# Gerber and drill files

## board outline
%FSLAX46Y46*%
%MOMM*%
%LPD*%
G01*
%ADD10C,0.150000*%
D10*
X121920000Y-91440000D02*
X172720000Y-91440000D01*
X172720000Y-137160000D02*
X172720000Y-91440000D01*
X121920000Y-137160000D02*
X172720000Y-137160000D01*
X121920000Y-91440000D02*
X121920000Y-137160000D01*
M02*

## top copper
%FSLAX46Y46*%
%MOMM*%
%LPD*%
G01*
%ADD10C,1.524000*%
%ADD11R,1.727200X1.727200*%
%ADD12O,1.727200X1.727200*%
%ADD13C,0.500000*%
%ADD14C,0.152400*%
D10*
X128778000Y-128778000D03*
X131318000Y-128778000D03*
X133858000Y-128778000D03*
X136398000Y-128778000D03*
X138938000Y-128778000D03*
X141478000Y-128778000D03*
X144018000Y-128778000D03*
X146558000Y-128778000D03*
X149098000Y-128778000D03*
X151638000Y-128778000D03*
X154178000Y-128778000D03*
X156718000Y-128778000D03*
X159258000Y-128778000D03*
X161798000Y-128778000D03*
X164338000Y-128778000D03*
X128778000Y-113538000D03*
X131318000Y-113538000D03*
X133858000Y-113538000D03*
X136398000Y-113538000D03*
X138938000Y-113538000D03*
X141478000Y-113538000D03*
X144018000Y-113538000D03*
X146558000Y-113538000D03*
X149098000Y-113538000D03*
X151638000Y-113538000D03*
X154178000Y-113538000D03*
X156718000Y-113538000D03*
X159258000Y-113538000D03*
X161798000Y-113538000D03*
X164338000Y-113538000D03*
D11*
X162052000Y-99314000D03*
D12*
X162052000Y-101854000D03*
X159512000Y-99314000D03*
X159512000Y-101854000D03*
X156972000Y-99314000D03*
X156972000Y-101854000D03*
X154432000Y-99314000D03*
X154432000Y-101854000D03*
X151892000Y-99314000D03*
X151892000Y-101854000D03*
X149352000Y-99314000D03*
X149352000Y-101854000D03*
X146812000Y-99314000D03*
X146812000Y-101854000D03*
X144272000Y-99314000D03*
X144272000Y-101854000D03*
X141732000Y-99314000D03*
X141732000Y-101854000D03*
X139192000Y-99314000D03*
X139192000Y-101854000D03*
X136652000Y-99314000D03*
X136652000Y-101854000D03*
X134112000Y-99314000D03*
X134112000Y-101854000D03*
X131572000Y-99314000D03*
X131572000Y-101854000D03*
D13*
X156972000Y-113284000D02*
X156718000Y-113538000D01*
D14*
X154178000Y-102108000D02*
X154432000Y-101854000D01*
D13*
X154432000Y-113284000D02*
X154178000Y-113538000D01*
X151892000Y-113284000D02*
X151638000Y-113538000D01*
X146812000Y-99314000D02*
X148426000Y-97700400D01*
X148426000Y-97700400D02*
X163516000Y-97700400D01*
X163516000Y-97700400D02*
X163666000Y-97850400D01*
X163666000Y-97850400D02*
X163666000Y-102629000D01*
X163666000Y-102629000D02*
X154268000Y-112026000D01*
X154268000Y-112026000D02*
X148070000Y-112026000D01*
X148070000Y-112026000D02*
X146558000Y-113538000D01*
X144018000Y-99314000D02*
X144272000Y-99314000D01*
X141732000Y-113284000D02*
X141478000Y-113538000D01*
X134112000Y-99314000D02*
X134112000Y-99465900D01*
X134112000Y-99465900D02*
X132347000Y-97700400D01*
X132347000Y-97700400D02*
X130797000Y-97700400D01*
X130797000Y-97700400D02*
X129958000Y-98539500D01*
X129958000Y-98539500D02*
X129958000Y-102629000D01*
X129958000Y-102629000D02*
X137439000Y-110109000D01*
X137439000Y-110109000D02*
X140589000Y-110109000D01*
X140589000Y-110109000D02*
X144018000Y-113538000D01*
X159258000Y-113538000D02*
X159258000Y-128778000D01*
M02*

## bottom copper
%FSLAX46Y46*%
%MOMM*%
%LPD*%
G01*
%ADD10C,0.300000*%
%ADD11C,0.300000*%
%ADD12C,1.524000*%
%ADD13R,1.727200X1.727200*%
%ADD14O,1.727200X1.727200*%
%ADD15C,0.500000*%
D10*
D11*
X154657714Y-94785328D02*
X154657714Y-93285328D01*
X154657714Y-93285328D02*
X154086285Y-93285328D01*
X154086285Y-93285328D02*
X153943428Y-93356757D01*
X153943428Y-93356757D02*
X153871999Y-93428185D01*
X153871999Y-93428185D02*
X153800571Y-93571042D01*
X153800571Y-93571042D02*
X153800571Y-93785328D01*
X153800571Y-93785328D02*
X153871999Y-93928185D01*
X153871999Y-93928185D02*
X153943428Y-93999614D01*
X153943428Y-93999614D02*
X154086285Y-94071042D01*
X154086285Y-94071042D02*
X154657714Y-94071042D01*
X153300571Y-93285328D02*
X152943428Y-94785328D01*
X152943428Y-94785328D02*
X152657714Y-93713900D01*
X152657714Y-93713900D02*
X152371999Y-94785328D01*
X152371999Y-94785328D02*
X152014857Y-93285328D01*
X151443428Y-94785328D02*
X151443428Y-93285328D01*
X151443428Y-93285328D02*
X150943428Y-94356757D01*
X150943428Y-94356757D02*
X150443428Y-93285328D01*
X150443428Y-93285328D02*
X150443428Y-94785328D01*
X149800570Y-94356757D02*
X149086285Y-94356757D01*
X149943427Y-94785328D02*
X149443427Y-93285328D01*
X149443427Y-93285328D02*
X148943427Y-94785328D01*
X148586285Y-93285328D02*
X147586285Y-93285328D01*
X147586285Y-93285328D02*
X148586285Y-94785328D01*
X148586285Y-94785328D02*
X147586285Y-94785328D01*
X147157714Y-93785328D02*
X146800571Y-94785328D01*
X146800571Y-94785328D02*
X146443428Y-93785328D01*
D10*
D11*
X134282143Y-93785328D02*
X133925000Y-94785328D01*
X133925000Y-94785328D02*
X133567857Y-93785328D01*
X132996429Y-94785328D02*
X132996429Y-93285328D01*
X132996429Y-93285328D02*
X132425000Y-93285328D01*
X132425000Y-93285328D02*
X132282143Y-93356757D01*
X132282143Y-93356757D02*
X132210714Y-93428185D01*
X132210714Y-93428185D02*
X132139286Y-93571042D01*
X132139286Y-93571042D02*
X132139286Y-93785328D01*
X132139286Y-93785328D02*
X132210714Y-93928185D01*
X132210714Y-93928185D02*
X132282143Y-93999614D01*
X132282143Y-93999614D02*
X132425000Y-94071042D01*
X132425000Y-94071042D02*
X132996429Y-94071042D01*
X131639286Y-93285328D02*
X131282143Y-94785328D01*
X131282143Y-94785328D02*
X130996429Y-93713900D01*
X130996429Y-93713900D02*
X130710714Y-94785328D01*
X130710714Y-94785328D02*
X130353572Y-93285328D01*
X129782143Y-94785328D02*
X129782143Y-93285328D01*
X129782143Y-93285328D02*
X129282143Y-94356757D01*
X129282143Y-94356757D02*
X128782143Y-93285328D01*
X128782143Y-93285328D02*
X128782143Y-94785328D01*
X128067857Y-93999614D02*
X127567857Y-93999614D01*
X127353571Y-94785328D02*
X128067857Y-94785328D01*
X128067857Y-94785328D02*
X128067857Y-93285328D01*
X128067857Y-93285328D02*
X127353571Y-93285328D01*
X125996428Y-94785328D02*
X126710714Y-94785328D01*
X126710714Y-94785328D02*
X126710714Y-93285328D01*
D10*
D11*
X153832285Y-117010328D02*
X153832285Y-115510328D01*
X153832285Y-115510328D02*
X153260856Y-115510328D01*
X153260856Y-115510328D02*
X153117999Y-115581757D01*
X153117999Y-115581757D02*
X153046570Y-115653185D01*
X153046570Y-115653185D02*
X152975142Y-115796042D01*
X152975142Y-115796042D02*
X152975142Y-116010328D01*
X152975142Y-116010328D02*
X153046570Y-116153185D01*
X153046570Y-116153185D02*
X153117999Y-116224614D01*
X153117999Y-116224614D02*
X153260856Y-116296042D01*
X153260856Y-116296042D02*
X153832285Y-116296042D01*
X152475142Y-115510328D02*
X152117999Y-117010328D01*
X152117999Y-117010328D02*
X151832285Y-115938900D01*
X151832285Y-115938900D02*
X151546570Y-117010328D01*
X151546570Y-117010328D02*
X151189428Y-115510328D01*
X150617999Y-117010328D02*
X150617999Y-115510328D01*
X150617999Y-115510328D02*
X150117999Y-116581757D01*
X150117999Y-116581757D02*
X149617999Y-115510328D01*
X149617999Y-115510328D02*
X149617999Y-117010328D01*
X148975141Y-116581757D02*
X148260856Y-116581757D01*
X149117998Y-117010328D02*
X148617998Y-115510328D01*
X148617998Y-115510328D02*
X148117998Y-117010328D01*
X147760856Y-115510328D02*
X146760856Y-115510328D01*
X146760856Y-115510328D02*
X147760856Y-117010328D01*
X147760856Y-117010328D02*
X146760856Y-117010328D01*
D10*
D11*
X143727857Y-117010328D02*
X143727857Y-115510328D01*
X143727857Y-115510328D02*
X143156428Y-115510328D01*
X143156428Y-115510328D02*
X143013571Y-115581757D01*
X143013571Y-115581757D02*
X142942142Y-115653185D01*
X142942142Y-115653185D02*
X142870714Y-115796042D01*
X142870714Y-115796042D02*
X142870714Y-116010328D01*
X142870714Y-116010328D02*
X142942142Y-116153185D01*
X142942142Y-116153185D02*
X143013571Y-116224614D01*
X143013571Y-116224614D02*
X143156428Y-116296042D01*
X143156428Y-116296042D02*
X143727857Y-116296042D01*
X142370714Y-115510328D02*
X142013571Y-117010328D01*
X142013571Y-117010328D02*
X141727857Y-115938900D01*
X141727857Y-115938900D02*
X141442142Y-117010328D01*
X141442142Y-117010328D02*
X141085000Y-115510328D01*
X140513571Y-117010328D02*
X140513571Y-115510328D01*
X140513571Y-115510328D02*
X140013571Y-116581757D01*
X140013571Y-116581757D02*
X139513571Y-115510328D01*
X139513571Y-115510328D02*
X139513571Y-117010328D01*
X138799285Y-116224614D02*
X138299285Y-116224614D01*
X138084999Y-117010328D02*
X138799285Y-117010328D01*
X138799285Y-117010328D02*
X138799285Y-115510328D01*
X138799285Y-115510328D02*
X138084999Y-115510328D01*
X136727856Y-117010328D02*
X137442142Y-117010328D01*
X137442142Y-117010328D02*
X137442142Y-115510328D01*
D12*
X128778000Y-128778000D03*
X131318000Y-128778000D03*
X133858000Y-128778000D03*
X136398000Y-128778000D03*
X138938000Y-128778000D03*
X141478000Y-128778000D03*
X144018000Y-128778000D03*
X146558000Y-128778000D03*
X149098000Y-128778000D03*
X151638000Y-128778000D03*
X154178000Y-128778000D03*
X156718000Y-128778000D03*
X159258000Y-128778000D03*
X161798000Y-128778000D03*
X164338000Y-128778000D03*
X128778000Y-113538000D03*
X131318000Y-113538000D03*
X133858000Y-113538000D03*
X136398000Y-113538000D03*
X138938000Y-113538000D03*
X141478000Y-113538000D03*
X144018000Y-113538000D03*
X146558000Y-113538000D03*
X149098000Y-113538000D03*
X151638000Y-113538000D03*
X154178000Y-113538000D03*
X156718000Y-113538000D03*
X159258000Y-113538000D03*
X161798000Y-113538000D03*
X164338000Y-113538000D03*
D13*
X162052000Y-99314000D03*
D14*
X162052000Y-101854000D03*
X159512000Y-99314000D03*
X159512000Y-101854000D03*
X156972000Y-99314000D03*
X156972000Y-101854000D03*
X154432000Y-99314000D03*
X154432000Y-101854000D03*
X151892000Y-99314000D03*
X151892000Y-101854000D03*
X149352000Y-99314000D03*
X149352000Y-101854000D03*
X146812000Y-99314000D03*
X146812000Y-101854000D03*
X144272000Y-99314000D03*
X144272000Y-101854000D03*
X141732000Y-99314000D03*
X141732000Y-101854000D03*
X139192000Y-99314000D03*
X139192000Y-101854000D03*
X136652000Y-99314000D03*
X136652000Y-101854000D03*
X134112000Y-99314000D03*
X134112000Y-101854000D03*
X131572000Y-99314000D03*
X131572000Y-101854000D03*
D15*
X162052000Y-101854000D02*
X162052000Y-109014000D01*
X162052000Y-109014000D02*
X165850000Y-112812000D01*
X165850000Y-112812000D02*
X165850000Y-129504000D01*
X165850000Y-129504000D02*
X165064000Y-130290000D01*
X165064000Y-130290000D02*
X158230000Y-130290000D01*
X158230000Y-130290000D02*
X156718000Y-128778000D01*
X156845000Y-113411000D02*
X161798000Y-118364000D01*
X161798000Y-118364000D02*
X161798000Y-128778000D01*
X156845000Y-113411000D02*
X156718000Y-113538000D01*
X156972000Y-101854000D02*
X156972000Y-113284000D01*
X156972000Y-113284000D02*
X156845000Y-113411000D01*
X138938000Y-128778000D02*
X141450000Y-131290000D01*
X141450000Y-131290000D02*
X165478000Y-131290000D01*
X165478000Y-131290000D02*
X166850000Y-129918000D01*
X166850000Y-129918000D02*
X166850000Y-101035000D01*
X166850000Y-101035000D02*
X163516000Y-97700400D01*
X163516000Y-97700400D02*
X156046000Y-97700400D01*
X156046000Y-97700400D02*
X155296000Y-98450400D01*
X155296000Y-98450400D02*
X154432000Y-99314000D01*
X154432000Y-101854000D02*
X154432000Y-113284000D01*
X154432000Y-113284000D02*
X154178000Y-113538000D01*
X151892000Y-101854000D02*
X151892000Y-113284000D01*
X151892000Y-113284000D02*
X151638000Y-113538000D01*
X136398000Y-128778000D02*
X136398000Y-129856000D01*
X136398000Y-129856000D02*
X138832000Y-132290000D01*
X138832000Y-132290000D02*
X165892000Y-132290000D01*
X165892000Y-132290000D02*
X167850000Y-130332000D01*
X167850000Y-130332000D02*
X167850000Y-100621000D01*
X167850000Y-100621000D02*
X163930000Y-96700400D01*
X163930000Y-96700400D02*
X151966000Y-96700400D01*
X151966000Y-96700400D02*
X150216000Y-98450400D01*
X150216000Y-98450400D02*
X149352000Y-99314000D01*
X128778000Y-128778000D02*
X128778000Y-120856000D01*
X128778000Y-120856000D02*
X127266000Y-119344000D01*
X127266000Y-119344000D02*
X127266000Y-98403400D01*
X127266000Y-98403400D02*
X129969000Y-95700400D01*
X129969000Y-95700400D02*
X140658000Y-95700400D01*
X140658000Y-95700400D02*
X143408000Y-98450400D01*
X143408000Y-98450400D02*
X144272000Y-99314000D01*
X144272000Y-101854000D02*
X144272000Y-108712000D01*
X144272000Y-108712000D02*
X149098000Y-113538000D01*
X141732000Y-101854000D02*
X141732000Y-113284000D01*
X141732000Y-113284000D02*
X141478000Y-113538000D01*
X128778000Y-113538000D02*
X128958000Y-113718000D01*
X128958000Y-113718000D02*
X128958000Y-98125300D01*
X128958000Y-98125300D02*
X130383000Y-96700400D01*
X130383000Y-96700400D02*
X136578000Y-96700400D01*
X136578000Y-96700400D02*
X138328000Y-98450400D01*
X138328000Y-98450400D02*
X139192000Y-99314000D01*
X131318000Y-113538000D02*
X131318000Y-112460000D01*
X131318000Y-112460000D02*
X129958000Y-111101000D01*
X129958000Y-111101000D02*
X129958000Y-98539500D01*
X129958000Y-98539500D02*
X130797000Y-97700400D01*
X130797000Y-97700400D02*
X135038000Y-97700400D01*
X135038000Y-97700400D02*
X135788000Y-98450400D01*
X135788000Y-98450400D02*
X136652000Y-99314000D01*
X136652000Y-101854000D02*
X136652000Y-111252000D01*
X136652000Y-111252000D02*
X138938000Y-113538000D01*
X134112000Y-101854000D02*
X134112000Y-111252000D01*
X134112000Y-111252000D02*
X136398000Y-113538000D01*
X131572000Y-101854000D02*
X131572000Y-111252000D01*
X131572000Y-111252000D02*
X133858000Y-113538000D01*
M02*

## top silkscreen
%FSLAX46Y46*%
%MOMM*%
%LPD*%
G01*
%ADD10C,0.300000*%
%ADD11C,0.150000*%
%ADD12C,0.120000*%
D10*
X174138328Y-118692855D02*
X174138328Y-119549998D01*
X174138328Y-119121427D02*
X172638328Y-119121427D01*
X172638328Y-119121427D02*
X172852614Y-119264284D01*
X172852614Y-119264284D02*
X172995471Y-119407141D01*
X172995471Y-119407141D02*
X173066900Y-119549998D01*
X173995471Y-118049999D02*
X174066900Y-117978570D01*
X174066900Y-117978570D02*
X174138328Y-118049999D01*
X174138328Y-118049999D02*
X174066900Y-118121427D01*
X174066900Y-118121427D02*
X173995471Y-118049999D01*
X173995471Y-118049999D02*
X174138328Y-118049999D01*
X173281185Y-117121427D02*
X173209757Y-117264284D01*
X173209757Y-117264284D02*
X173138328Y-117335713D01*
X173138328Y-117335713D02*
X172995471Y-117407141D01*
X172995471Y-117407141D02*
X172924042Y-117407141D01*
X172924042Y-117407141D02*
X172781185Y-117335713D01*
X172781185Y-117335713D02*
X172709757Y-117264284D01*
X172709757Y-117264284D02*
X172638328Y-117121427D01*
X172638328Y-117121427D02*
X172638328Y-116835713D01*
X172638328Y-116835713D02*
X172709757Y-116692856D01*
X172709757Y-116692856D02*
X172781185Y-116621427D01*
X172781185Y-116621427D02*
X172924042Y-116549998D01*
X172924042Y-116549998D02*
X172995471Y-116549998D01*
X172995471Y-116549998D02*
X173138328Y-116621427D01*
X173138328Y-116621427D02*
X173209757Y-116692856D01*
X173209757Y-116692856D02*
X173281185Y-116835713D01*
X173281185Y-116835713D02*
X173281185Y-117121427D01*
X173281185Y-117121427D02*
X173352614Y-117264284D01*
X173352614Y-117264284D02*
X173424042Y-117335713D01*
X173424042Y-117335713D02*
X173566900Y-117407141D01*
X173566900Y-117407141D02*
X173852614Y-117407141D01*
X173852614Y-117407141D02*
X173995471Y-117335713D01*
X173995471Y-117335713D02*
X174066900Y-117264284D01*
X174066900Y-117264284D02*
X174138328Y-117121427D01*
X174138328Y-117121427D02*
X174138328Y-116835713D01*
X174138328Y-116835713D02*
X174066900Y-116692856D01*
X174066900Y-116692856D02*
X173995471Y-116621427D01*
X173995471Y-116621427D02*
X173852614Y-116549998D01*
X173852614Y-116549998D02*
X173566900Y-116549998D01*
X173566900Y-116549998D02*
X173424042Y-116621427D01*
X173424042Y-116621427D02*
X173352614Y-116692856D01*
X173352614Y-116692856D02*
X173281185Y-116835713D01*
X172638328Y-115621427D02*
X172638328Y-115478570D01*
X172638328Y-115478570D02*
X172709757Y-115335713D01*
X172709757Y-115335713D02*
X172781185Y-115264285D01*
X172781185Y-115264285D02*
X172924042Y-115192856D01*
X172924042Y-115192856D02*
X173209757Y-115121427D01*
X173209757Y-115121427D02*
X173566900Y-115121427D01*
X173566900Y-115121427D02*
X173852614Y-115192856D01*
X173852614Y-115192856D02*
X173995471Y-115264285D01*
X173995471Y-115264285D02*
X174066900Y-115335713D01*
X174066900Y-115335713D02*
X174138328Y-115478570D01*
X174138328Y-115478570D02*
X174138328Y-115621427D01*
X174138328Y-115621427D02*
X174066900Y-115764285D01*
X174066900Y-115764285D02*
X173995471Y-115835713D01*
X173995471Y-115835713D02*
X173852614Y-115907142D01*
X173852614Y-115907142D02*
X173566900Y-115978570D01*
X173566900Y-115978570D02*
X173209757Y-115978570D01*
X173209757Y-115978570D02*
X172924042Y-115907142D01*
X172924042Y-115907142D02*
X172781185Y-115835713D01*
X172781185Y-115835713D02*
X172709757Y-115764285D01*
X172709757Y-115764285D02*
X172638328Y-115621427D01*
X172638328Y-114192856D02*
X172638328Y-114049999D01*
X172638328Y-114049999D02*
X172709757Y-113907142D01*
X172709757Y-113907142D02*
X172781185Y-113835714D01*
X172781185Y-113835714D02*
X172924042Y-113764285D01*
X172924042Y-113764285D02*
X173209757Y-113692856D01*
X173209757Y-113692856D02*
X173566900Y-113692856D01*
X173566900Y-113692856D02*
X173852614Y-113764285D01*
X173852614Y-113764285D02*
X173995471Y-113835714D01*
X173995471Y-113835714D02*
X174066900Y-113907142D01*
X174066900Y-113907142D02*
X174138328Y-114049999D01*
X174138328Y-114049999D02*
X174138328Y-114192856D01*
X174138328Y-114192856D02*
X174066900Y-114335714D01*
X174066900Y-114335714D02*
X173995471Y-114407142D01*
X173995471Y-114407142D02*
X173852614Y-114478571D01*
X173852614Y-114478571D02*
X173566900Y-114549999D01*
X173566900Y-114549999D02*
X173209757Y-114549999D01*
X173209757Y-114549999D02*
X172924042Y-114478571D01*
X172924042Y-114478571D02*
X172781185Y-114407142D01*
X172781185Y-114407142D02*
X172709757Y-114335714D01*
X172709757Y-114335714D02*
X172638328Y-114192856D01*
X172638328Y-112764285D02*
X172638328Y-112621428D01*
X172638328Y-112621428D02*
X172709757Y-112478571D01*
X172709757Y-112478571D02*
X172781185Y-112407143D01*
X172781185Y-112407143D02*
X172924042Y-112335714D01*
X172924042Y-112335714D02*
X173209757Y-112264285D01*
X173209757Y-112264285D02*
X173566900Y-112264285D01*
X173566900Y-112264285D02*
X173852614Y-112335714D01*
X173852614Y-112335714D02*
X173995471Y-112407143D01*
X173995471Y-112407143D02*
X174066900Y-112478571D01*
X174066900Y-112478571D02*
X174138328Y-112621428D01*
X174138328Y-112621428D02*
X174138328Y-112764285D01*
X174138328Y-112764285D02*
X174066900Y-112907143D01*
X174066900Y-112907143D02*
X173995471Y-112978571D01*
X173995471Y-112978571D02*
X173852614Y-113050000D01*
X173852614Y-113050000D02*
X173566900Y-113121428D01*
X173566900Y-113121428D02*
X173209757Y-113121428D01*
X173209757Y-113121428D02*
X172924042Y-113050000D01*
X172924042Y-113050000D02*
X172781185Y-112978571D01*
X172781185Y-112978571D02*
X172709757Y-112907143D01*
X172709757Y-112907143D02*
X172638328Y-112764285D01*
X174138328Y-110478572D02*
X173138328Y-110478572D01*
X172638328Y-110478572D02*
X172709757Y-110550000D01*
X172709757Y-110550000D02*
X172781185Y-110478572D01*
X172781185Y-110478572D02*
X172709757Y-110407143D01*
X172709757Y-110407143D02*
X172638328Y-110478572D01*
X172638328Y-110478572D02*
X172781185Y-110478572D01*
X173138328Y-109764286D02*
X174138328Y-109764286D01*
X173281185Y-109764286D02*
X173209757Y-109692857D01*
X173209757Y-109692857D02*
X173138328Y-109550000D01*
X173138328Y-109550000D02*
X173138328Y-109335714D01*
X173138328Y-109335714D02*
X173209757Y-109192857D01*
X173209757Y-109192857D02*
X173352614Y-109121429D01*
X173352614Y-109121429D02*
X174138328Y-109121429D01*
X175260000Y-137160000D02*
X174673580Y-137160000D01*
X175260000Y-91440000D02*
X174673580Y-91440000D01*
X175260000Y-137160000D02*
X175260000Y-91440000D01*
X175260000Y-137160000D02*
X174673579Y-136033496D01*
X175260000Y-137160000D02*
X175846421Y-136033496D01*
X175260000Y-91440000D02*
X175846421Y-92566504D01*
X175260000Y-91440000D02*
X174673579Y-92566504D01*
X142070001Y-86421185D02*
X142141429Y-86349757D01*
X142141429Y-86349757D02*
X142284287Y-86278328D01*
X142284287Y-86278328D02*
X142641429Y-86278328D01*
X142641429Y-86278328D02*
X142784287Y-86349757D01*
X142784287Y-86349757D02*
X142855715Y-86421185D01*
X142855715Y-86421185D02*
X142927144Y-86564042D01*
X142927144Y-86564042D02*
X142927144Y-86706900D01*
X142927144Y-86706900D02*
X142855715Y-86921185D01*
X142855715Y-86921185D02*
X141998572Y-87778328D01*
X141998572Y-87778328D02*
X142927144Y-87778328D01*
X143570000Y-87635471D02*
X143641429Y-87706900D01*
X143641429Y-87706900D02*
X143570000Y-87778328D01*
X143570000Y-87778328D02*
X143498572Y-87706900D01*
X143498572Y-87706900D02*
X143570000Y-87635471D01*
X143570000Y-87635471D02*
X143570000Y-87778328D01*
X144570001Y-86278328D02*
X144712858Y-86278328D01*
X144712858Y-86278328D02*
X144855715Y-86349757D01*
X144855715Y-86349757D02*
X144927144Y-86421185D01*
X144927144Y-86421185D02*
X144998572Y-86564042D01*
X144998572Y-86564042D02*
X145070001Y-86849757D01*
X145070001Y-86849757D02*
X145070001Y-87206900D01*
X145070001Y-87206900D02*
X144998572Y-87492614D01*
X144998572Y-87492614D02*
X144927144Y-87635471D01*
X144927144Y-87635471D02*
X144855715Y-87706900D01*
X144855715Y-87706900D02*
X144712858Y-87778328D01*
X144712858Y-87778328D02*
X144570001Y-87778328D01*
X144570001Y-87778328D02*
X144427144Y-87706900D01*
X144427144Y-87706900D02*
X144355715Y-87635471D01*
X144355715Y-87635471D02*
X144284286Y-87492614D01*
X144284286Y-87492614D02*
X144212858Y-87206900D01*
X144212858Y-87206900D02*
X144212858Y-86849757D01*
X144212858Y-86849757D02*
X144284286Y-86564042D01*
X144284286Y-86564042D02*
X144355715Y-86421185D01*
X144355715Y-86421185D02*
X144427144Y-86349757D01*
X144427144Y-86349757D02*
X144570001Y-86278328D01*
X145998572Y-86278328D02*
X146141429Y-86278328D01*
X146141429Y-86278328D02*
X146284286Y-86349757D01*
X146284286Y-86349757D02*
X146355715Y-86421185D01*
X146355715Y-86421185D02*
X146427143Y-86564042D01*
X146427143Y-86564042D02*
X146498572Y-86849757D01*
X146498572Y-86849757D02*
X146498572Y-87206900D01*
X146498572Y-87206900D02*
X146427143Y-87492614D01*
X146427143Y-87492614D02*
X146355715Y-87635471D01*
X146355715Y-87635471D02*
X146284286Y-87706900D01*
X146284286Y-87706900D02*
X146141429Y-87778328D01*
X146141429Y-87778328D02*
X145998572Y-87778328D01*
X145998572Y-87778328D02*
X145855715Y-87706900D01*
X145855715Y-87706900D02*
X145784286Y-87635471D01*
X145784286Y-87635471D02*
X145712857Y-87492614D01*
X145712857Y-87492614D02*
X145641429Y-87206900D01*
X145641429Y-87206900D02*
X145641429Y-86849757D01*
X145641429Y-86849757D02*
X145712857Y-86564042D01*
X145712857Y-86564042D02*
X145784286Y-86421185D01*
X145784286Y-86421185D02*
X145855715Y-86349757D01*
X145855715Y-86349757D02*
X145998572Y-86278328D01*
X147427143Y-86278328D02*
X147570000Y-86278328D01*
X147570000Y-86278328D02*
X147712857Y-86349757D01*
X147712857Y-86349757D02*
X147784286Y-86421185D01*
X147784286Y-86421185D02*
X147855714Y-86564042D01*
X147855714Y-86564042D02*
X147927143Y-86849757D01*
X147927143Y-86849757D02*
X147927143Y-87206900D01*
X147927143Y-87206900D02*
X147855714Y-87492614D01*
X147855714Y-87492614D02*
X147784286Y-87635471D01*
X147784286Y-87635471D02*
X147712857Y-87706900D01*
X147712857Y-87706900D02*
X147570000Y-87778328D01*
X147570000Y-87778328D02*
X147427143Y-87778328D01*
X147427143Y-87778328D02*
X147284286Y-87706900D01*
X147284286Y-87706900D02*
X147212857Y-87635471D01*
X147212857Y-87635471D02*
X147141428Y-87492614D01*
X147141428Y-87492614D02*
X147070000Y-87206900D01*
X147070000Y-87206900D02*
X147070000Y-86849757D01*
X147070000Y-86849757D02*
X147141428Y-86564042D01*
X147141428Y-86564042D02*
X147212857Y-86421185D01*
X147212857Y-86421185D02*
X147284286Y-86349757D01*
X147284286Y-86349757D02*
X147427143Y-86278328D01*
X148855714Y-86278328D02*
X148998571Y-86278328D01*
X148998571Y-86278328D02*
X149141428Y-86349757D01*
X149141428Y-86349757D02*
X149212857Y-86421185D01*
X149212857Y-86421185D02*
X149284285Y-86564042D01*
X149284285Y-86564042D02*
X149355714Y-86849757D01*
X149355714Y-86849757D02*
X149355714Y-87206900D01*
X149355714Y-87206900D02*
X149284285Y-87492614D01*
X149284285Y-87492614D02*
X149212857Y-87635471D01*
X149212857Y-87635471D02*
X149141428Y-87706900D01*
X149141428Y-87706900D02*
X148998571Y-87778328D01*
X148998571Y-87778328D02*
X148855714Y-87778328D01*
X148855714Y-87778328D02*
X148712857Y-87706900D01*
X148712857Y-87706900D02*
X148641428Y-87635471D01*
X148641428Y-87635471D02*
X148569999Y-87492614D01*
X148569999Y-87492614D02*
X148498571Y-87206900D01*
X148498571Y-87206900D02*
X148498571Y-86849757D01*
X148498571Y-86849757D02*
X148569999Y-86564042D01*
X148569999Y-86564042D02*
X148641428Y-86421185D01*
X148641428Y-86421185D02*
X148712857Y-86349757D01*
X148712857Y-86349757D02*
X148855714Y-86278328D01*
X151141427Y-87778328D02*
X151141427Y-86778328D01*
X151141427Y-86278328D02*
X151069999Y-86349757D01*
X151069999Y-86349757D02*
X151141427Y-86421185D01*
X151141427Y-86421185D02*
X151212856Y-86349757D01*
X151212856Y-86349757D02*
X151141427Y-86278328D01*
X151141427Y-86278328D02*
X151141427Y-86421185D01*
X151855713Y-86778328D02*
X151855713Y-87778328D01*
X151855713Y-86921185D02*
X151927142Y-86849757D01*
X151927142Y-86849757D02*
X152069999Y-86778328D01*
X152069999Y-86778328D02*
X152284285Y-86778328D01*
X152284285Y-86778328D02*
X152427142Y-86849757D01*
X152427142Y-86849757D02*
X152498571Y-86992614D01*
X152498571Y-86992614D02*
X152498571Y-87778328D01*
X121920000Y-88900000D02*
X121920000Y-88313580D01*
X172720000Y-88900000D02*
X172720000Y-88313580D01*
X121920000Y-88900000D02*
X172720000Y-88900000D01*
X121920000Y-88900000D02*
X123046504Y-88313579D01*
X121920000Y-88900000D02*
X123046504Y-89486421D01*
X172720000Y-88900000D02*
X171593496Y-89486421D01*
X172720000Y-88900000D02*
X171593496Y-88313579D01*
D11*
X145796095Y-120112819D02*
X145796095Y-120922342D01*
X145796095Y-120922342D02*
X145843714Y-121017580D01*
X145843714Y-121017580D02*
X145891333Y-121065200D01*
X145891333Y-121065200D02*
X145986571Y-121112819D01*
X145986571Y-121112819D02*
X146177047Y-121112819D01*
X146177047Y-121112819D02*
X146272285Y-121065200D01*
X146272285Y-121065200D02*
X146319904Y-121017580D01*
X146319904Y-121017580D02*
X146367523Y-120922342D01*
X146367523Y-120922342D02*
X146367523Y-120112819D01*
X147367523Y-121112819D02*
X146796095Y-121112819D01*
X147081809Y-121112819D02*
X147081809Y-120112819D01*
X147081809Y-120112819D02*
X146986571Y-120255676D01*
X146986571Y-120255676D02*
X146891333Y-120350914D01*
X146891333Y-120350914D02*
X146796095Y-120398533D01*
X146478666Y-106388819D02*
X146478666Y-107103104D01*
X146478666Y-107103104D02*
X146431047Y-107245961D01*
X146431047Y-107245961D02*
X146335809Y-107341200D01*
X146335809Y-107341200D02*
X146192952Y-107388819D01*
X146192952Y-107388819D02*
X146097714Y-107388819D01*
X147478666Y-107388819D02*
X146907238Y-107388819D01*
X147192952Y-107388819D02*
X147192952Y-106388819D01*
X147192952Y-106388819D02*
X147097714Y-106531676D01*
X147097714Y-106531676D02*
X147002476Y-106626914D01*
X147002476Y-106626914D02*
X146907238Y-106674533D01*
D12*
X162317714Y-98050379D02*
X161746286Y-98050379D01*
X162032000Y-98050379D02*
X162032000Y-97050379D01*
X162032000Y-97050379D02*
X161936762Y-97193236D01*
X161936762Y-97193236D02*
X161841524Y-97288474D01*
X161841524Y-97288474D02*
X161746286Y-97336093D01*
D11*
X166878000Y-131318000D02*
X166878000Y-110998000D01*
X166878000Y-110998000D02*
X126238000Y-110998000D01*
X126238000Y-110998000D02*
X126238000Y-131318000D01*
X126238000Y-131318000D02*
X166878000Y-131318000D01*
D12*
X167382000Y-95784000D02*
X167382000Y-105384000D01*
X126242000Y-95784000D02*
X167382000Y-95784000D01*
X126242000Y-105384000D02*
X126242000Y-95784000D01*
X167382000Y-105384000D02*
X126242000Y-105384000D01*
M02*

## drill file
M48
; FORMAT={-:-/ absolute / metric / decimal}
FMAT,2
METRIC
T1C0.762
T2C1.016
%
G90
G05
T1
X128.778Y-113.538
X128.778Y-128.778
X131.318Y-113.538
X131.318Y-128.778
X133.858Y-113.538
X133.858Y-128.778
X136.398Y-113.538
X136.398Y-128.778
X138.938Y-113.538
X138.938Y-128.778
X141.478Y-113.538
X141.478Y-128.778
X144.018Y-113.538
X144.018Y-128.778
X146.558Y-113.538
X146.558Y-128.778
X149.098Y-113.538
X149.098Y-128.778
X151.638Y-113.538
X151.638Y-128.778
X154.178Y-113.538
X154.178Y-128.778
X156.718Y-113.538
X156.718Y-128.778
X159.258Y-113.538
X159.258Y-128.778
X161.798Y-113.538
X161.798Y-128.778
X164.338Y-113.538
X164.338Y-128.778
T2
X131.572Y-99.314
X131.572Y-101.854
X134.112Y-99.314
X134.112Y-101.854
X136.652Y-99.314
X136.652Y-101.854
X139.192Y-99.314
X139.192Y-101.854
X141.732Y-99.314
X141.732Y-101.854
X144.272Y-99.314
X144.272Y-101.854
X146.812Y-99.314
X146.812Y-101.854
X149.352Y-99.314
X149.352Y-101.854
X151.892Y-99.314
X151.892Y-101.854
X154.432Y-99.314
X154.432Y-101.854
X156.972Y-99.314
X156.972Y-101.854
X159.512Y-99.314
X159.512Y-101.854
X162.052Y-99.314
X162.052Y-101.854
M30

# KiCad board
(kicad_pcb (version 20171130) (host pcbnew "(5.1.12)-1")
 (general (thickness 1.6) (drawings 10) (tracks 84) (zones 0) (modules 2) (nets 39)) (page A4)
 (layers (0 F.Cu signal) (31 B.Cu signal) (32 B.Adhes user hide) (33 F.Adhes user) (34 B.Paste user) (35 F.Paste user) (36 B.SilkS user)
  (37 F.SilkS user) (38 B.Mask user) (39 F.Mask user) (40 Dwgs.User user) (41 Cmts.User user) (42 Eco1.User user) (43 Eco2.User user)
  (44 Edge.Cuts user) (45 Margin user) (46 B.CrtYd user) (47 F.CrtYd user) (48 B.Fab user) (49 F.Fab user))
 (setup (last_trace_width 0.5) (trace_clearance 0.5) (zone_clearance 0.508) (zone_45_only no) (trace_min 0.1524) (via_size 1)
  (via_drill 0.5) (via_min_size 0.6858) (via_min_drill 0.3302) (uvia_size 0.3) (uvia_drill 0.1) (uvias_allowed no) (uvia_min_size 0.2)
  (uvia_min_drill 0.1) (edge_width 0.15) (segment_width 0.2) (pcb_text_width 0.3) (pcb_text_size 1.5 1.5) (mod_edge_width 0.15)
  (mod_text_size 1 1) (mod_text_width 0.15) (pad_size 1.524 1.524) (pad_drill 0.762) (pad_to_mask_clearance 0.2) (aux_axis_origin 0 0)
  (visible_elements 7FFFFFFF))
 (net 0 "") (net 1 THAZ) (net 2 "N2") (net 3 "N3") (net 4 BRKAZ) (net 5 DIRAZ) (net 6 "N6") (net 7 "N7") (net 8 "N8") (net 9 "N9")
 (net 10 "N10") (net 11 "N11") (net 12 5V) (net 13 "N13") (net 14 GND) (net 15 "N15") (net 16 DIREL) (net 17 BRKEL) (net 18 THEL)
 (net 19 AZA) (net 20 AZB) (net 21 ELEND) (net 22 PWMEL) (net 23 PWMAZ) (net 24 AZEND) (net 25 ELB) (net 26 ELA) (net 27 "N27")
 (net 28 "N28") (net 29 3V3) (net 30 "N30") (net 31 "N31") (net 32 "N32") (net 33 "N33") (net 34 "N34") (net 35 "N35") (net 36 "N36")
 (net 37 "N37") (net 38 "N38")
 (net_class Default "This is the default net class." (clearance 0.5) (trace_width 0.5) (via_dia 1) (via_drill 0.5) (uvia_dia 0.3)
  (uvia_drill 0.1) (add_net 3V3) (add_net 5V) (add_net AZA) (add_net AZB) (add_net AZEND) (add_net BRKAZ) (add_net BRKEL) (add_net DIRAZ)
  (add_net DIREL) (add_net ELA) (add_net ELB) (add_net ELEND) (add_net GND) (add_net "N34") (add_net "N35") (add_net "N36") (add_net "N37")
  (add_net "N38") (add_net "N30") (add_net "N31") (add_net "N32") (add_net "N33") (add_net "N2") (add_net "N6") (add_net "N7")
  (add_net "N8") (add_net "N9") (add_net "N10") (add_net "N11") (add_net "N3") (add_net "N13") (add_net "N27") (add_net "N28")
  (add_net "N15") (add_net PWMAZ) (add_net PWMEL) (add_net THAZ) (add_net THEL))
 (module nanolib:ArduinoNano (layer F.Cu) (at 146.558 121.158 180)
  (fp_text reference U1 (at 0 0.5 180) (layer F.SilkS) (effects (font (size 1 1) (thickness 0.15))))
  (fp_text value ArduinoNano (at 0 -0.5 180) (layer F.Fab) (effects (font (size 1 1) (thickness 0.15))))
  (fp_line (start -20.32 -10.16) (end -20.32 10.16) (layer F.SilkS) (width 0.15))
  (fp_line (start -20.32 10.16) (end 20.32 10.16) (layer F.SilkS) (width 0.15))
  (fp_line (start 20.32 10.16) (end 20.32 -10.16) (layer F.SilkS) (width 0.15))
  (fp_line (start 20.32 -10.16) (end -20.32 -10.16) (layer F.SilkS) (width 0.15))
  (pad D13 thru_hole circle (at 17.78 -7.62 180) (size 1.524 1.524) (drill 0.762) (layers *.Cu *.Mask) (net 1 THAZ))
  (pad 3V3 thru_hole circle (at 15.24 -7.62 180) (size 1.524 1.524) (drill 0.762) (layers *.Cu *.Mask) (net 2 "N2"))
  (pad REF thru_hole circle (at 12.7 -7.62 180) (size 1.524 1.524) (drill 0.762) (layers *.Cu *.Mask) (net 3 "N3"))
  (pad A0 thru_hole circle (at 10.16 -7.62 180) (size 1.524 1.524) (drill 0.762) (layers *.Cu *.Mask) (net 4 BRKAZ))
  (pad A1 thru_hole circle (at 7.62 -7.62 180) (size 1.524 1.524) (drill 0.762) (layers *.Cu *.Mask) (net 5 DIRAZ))
  (pad A2 thru_hole circle (at 5.08 -7.62 180) (size 1.524 1.524) (drill 0.762) (layers *.Cu *.Mask) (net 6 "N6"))
  (pad A3 thru_hole circle (at 2.54 -7.62 180) (size 1.524 1.524) (drill 0.762) (layers *.Cu *.Mask) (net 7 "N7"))
  (pad A4 thru_hole circle (at 0 -7.62 180) (size 1.524 1.524) (drill 0.762) (layers *.Cu *.Mask) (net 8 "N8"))
  (pad A5 thru_hole circle (at -2.54 -7.62 180) (size 1.524 1.524) (drill 0.762) (layers *.Cu *.Mask) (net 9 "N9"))
  (pad A6 thru_hole circle (at -5.08 -7.62 180) (size 1.524 1.524) (drill 0.762) (layers *.Cu *.Mask) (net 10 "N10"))
  (pad A7 thru_hole circle (at -7.62 -7.62 180) (size 1.524 1.524) (drill 0.762) (layers *.Cu *.Mask) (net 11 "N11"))
  (pad 5V thru_hole circle (at -10.16 -7.62 180) (size 1.524 1.524) (drill 0.762) (layers *.Cu *.Mask) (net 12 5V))
  (pad RST thru_hole circle (at -12.7 -7.62 180) (size 1.524 1.524) (drill 0.762) (layers *.Cu *.Mask) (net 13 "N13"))
  (pad GND thru_hole circle (at -15.24 -7.62 180) (size 1.524 1.524) (drill 0.762) (layers *.Cu *.Mask) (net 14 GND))
  (pad VIN thru_hole circle (at -17.78 -7.62 180) (size 1.524 1.524) (drill 0.762) (layers *.Cu *.Mask) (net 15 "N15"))
  (pad D12 thru_hole circle (at 17.78 7.62 180) (size 1.524 1.524) (drill 0.762) (layers *.Cu *.Mask) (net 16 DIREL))
  (pad D11 thru_hole circle (at 15.24 7.62 180) (size 1.524 1.524) (drill 0.762) (layers *.Cu *.Mask) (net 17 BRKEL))
  (pad D10 thru_hole circle (at 12.7 7.62 180) (size 1.524 1.524) (drill 0.762) (layers *.Cu *.Mask) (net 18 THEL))
  (pad D9 thru_hole circle (at 10.16 7.62 180) (size 1.524 1.524) (drill 0.762) (layers *.Cu *.Mask) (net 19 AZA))
  (pad D8 thru_hole circle (at 7.62 7.62 180) (size 1.524 1.524) (drill 0.762) (layers *.Cu *.Mask) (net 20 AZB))
  (pad D7 thru_hole circle (at 5.08 7.62 180) (size 1.524 1.524) (drill 0.762) (layers *.Cu *.Mask) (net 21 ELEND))
  (pad D6 thru_hole circle (at 2.54 7.62 180) (size 1.524 1.524) (drill 0.762) (layers *.Cu *.Mask) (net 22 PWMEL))
  (pad D5 thru_hole circle (at 0 7.62 180) (size 1.524 1.524) (drill 0.762) (layers *.Cu *.Mask) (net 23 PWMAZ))
  (pad D4 thru_hole circle (at -2.54 7.62 180) (size 1.524 1.524) (drill 0.762) (layers *.Cu *.Mask) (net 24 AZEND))
  (pad D3 thru_hole circle (at -5.08 7.62 180) (size 1.524 1.524) (drill 0.762) (layers *.Cu *.Mask) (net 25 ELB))
  (pad D2 thru_hole circle (at -7.62 7.62 180) (size 1.524 1.524) (drill 0.762) (layers *.Cu *.Mask) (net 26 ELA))
  (pad GND thru_hole circle (at -10.16 7.62 180) (size 1.524 1.524) (drill 0.762) (layers *.Cu *.Mask) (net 14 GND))
  (pad RST thru_hole circle (at -12.7 7.62 180) (size 1.524 1.524) (drill 0.762) (layers *.Cu *.Mask) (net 13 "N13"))
  (pad RX0 thru_hole circle (at -15.24 7.62 180) (size 1.524 1.524) (drill 0.762) (layers *.Cu *.Mask) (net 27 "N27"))
  (pad TX1 thru_hole circle (at -17.78 7.62 180) (size 1.524 1.524) (drill 0.762) (layers *.Cu *.Mask) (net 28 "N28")))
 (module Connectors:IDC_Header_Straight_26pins (layer F.Cu) (at 162.052 99.314 180)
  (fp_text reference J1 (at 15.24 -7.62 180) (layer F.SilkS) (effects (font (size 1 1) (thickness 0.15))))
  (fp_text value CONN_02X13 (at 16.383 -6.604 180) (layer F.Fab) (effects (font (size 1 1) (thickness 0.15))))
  (fp_line (start -5.33 3.53) (end -5.33 -6.07) (layer F.SilkS) (width 0.12))
  (fp_line (start 35.81 3.53) (end -5.33 3.53) (layer F.SilkS) (width 0.12))
  (fp_line (start 35.81 -6.07) (end 35.81 3.53) (layer F.SilkS) (width 0.12))
  (fp_line (start -5.33 -6.07) (end 35.81 -6.07) (layer F.SilkS) (width 0.12))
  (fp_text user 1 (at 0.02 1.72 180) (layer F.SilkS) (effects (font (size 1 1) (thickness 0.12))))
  (pad 1 thru_hole rect (at 0 0 180) (size 1.7272 1.7272) (drill 1.016) (layers *.Cu *.Mask) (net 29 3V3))
  (pad 2 thru_hole oval (at 0 -2.54 180) (size 1.7272 1.7272) (drill 1.016) (layers *.Cu *.Mask) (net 12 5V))
  (pad 3 thru_hole oval (at 2.54 0 180) (size 1.7272 1.7272) (drill 1.016) (layers *.Cu *.Mask) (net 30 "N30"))
  (pad 4 thru_hole oval (at 2.54 -2.54 180) (size 1.7272 1.7272) (drill 1.016) (layers *.Cu *.Mask) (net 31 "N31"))
  (pad 5 thru_hole oval (at 5.08 0 180) (size 1.7272 1.7272) (drill 1.016) (layers *.Cu *.Mask) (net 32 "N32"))
  (pad 6 thru_hole oval (at 5.08 -2.54 180) (size 1.7272 1.7272) (drill 1.016) (layers *.Cu *.Mask) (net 14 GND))
  (pad 7 thru_hole oval (at 7.62 0 180) (size 1.7272 1.7272) (drill 1.016) (layers *.Cu *.Mask) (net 5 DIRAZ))
  (pad 8 thru_hole oval (at 7.62 -2.54 180) (size 1.7272 1.7272) (drill 1.016) (layers *.Cu *.Mask) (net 26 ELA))
  (pad 9 thru_hole oval (at 10.16 0 180) (size 1.7272 1.7272) (drill 1.016) (layers *.Cu *.Mask) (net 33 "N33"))
  (pad 10 thru_hole oval (at 10.16 -2.54 180) (size 1.7272 1.7272) (drill 1.016) (layers *.Cu *.Mask) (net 25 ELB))
  (pad 11 thru_hole oval (at 12.7 0 180) (size 1.7272 1.7272) (drill 1.016) (layers *.Cu *.Mask) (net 4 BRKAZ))
  (pad 12 thru_hole oval (at 12.7 -2.54 180) (size 1.7272 1.7272) (drill 1.016) (layers *.Cu *.Mask) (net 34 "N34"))
  (pad 13 thru_hole oval (at 15.24 0 180) (size 1.7272 1.7272) (drill 1.016) (layers *.Cu *.Mask) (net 23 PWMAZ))
  (pad 14 thru_hole oval (at 15.24 -2.54 180) (size 1.7272 1.7272) (drill 1.016) (layers *.Cu *.Mask) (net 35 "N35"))
  (pad 15 thru_hole oval (at 17.78 0 180) (size 1.7272 1.7272) (drill 1.016) (layers *.Cu *.Mask) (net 1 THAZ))
  (pad 16 thru_hole oval (at 17.78 -2.54 180) (size 1.7272 1.7272) (drill 1.016) (layers *.Cu *.Mask) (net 24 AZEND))
  (pad 17 thru_hole oval (at 20.32 0 180) (size 1.7272 1.7272) (drill 1.016) (layers *.Cu *.Mask) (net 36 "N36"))
  (pad 18 thru_hole oval (at 20.32 -2.54 180) (size 1.7272 1.7272) (drill 1.016) (layers *.Cu *.Mask) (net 21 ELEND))
  (pad 19 thru_hole oval (at 22.86 0 180) (size 1.7272 1.7272) (drill 1.016) (layers *.Cu *.Mask) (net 16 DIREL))
  (pad 20 thru_hole oval (at 22.86 -2.54 180) (size 1.7272 1.7272) (drill 1.016) (layers *.Cu *.Mask) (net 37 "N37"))
  (pad 21 thru_hole oval (at 25.4 0 180) (size 1.7272 1.7272) (drill 1.016) (layers *.Cu *.Mask) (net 17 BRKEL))
  (pad 22 thru_hole oval (at 25.4 -2.54 180) (size 1.7272 1.7272) (drill 1.016) (layers *.Cu *.Mask) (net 20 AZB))
  (pad 23 thru_hole oval (at 27.94 0 180) (size 1.7272 1.7272) (drill 1.016) (layers *.Cu *.Mask) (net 22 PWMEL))
  (pad 24 thru_hole oval (at 27.94 -2.54 180) (size 1.7272 1.7272) (drill 1.016) (layers *.Cu *.Mask) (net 19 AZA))
  (pad 25 thru_hole oval (at 30.48 0 180) (size 1.7272 1.7272) (drill 1.016) (layers *.Cu *.Mask) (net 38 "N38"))
  (pad 26 thru_hole oval (at 30.48 -2.54 180) (size 1.7272 1.7272) (drill 1.016) (layers *.Cu *.Mask) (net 18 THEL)))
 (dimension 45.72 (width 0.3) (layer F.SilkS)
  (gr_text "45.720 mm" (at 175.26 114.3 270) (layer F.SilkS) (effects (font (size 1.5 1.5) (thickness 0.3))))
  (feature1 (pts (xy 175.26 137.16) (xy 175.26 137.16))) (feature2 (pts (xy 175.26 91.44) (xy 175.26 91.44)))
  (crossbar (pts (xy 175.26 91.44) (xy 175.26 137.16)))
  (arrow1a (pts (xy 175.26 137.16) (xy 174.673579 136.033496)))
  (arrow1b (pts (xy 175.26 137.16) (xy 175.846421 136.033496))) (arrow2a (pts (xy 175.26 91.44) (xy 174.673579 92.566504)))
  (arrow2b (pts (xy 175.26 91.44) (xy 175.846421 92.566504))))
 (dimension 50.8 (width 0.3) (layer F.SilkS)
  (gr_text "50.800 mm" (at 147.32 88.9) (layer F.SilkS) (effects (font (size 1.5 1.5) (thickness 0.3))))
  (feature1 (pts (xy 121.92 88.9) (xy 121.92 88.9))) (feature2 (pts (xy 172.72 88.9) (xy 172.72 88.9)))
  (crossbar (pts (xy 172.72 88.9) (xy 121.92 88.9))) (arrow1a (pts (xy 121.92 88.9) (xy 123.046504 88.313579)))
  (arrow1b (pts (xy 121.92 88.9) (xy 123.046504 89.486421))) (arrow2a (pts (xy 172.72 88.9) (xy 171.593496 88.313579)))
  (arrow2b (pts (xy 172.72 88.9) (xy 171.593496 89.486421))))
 (gr_line (start 121.92 91.44) (end 172.72 91.44) (layer Edge.Cuts) (width 0.15))
 (gr_line (start 172.72 137.16) (end 172.72 91.44) (layer Edge.Cuts) (width 0.15))
 (gr_line (start 121.92 137.16) (end 172.72 137.16) (layer Edge.Cuts) (width 0.15))
 (gr_line (start 121.92 91.44) (end 121.92 137.16) (layer Edge.Cuts) (width 0.15))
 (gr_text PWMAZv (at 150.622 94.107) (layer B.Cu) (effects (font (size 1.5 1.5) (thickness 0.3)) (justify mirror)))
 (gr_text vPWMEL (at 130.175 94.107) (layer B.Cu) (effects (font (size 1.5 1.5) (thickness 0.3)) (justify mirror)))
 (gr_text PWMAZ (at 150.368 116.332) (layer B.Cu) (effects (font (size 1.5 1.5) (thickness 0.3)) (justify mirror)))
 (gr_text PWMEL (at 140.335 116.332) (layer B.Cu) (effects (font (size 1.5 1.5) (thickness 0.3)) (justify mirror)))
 (segment (start 162.052 101.854) (end 162.052 109.014) (width 0.5) (layer B.Cu) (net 12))
 (segment (start 162.052 109.014) (end 165.85 112.812) (width 0.5) (layer B.Cu) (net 12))
 (segment (start 165.85 112.812) (end 165.85 129.504) (width 0.5) (layer B.Cu) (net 12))
 (segment (start 165.85 129.504) (end 165.064 130.29) (width 0.5) (layer B.Cu) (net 12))
 (segment (start 165.064 130.29) (end 158.23 130.29) (width 0.5) (layer B.Cu) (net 12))
 (segment (start 158.23 130.29) (end 156.718 128.778) (width 0.5) (layer B.Cu) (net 12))
 (segment (start 156.845 113.411) (end 161.798 118.364) (width 0.5) (layer B.Cu) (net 14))
 (segment (start 161.798 118.364) (end 161.798 128.778) (width 0.5) (layer B.Cu) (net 14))
 (segment (start 156.845 113.411) (end 156.718 113.538) (width 0.5) (layer B.Cu) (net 14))
 (segment (start 156.972 101.854) (end 156.972 113.284) (width 0.5) (layer B.Cu) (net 14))
 (segment (start 156.972 113.284) (end 156.845 113.411) (width 0.5) (layer B.Cu) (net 14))
 (segment (start 156.972 113.284) (end 156.718 113.538) (width 0.5) (layer F.Cu) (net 14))
 (segment (start 138.938 128.778) (end 141.45 131.29) (width 0.5) (layer B.Cu) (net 5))
 (segment (start 141.45 131.29) (end 165.478 131.29) (width 0.5) (layer B.Cu) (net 5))
 (segment (start 165.478 131.29) (end 166.85 129.918) (width 0.5) (layer B.Cu) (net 5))
 (segment (start 166.85 129.918) (end 166.85 101.035) (width 0.5) (layer B.Cu) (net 5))
 (segment (start 166.85 101.035) (end 163.516 97.7004) (width 0.5) (layer B.Cu) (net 5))
 (segment (start 163.516 97.7004) (end 156.046 97.7004) (width 0.5) (layer B.Cu) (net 5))
 (segment (start 156.046 97.7004) (end 155.296 98.4504) (width 0.5) (layer B.Cu) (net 5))
 (segment (start 155.296 98.4504) (end 154.432 99.314) (width 0.5) (layer B.Cu) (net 5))
 (segment (start 154.178 102.108) (end 154.432 101.854) (width 0.1524) (layer F.Cu) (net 26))
 (segment (start 154.432 113.284) (end 154.178 113.538) (width 0.5) (layer F.Cu) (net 26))
 (segment (start 154.432 101.854) (end 154.432 113.284) (width 0.5) (layer B.Cu) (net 26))
 (segment (start 154.432 113.284) (end 154.178 113.538) (width 0.5) (layer B.Cu) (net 26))
 (segment (start 151.892 113.284) (end 151.638 113.538) (width 0.5) (layer F.Cu) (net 25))
 (segment (start 151.892 101.854) (end 151.892 113.284) (width 0.5) (layer B.Cu) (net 25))
 (segment (start 151.892 113.284) (end 151.638 113.538) (width 0.5) (layer B.Cu) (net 25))
 (segment (start 136.398 128.778) (end 136.398 129.856) (width 0.5) (layer B.Cu) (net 4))
 (segment (start 136.398 129.856) (end 138.832 132.29) (width 0.5) (layer B.Cu) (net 4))
 (segment (start 138.832 132.29) (end 165.892 132.29) (width 0.5) (layer B.Cu) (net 4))
 (segment (start 165.892 132.29) (end 167.85 130.332) (width 0.5) (layer B.Cu) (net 4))
 (segment (start 167.85 130.332) (end 167.85 100.621) (width 0.5) (layer B.Cu) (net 4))
 (segment (start 167.85 100.621) (end 163.93 96.7004) (width 0.5) (layer B.Cu) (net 4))
 (segment (start 163.93 96.7004) (end 151.966 96.7004) (width 0.5) (layer B.Cu) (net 4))
 (segment (start 151.966 96.7004) (end 150.216 98.4504) (width 0.5) (layer B.Cu) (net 4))
 (segment (start 150.216 98.4504) (end 149.352 99.314) (width 0.5) (layer B.Cu) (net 4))
 (segment (start 146.812 99.314) (end 148.426 97.7004) (width 0.5) (layer F.Cu) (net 23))
 (segment (start 148.426 97.7004) (end 163.516 97.7004) (width 0.5) (layer F.Cu) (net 23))
 (segment (start 163.516 97.7004) (end 163.666 97.8504) (width 0.5) (layer F.Cu) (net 23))
 (segment (start 163.666 97.8504) (end 163.666 102.629) (width 0.5) (layer F.Cu) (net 23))
 (segment (start 163.666 102.629) (end 154.268 112.026) (width 0.5) (layer F.Cu) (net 23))
 (segment (start 154.268 112.026) (end 148.07 112.026) (width 0.5) (layer F.Cu) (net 23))
 (segment (start 148.07 112.026) (end 146.558 113.538) (width 0.5) (layer F.Cu) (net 23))
 (segment (start 144.018 99.314) (end 144.272 99.314) (width 0.5) (layer F.Cu) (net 1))
 (segment (start 128.778 128.778) (end 128.778 120.856) (width 0.5) (layer B.Cu) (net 1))
 (segment (start 128.778 120.856) (end 127.266 119.344) (width 0.5) (layer B.Cu) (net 1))
 (segment (start 127.266 119.344) (end 127.266 98.4034) (width 0.5) (layer B.Cu) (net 1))
 (segment (start 127.266 98.4034) (end 129.969 95.7004) (width 0.5) (layer B.Cu) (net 1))
 (segment (start 129.969 95.7004) (end 140.658 95.7004) (width 0.5) (layer B.Cu) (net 1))
 (segment (start 140.658 95.7004) (end 143.408 98.4504) (width 0.5) (layer B.Cu) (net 1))
 (segment (start 143.408 98.4504) (end 144.272 99.314) (width 0.5) (layer B.Cu) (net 1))
 (segment (start 144.272 101.854) (end 144.272 108.712) (width 0.5) (layer B.Cu) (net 24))
 (segment (start 144.272 108.712) (end 149.098 113.538) (width 0.5) (layer B.Cu) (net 24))
 (segment (start 141.732 113.284) (end 141.478 113.538) (width 0.5) (layer F.Cu) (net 21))
 (segment (start 141.732 101.854) (end 141.732 113.284) (width 0.5) (layer B.Cu) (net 21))
 (segment (start 141.732 113.284) (end 141.478 113.538) (width 0.5) (layer B.Cu) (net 21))
 (segment (start 128.778 113.538) (end 128.958 113.718) (width 0.5) (layer B.Cu) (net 16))
 (segment (start 128.958 113.718) (end 128.958 98.1253) (width 0.5) (layer B.Cu) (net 16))
 (segment (start 128.958 98.1253) (end 130.383 96.7004) (width 0.5) (layer B.Cu) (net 16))
 (segment (start 130.383 96.7004) (end 136.578 96.7004) (width 0.5) (layer B.Cu) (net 16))
 (segment (start 136.578 96.7004) (end 138.328 98.4504) (width 0.5) (layer B.Cu) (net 16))
 (segment (start 138.328 98.4504) (end 139.192 99.314) (width 0.5) (layer B.Cu) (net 16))
 (segment (start 131.318 113.538) (end 131.318 112.46) (width 0.5) (layer B.Cu) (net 17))
 (segment (start 131.318 112.46) (end 129.958 111.101) (width 0.5) (layer B.Cu) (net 17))
 (segment (start 129.958 111.101) (end 129.958 98.5395) (width 0.5) (layer B.Cu) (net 17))
 (segment (start 129.958 98.5395) (end 130.797 97.7004) (width 0.5) (layer B.Cu) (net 17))
 (segment (start 130.797 97.7004) (end 135.038 97.7004) (width 0.5) (layer B.Cu) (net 17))
 (segment (start 135.038 97.7004) (end 135.788 98.4504) (width 0.5) (layer B.Cu) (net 17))
 (segment (start 135.788 98.4504) (end 136.652 99.314) (width 0.5) (layer B.Cu) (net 17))
 (segment (start 136.652 101.854) (end 136.652 111.252) (width 0.5) (layer B.Cu) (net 20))
 (segment (start 136.652 111.252) (end 138.938 113.538) (width 0.5) (layer B.Cu) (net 20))
 (segment (start 134.112 99.314) (end 134.112 99.4659) (width 0.5) (layer F.Cu) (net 22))
 (segment (start 134.112 99.4659) (end 132.347 97.7004) (width 0.5) (layer F.Cu) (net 22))
 (segment (start 132.347 97.7004) (end 130.797 97.7004) (width 0.5) (layer F.Cu) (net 22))
 (segment (start 130.797 97.7004) (end 129.958 98.5395) (width 0.5) (layer F.Cu) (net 22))
 (segment (start 129.958 98.5395) (end 129.958 102.629) (width 0.5) (layer F.Cu) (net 22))
 (segment (start 129.958 102.629) (end 137.439 110.109) (width 0.5) (layer F.Cu) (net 22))
 (segment (start 137.439 110.109) (end 140.589 110.109) (width 0.5) (layer F.Cu) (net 22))
 (segment (start 140.589 110.109) (end 144.018 113.538) (width 0.5) (layer F.Cu) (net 22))
 (segment (start 134.112 101.854) (end 134.112 111.252) (width 0.5) (layer B.Cu) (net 19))
 (segment (start 134.112 111.252) (end 136.398 113.538) (width 0.5) (layer B.Cu) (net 19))
 (segment (start 131.572 101.854) (end 131.572 111.252) (width 0.5) (layer B.Cu) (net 18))
 (segment (start 131.572 111.252) (end 133.858 113.538) (width 0.5) (layer B.Cu) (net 18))
 (segment (start 159.258 113.538) (end 159.258 128.778) (width 0.5) (layer F.Cu) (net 13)))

